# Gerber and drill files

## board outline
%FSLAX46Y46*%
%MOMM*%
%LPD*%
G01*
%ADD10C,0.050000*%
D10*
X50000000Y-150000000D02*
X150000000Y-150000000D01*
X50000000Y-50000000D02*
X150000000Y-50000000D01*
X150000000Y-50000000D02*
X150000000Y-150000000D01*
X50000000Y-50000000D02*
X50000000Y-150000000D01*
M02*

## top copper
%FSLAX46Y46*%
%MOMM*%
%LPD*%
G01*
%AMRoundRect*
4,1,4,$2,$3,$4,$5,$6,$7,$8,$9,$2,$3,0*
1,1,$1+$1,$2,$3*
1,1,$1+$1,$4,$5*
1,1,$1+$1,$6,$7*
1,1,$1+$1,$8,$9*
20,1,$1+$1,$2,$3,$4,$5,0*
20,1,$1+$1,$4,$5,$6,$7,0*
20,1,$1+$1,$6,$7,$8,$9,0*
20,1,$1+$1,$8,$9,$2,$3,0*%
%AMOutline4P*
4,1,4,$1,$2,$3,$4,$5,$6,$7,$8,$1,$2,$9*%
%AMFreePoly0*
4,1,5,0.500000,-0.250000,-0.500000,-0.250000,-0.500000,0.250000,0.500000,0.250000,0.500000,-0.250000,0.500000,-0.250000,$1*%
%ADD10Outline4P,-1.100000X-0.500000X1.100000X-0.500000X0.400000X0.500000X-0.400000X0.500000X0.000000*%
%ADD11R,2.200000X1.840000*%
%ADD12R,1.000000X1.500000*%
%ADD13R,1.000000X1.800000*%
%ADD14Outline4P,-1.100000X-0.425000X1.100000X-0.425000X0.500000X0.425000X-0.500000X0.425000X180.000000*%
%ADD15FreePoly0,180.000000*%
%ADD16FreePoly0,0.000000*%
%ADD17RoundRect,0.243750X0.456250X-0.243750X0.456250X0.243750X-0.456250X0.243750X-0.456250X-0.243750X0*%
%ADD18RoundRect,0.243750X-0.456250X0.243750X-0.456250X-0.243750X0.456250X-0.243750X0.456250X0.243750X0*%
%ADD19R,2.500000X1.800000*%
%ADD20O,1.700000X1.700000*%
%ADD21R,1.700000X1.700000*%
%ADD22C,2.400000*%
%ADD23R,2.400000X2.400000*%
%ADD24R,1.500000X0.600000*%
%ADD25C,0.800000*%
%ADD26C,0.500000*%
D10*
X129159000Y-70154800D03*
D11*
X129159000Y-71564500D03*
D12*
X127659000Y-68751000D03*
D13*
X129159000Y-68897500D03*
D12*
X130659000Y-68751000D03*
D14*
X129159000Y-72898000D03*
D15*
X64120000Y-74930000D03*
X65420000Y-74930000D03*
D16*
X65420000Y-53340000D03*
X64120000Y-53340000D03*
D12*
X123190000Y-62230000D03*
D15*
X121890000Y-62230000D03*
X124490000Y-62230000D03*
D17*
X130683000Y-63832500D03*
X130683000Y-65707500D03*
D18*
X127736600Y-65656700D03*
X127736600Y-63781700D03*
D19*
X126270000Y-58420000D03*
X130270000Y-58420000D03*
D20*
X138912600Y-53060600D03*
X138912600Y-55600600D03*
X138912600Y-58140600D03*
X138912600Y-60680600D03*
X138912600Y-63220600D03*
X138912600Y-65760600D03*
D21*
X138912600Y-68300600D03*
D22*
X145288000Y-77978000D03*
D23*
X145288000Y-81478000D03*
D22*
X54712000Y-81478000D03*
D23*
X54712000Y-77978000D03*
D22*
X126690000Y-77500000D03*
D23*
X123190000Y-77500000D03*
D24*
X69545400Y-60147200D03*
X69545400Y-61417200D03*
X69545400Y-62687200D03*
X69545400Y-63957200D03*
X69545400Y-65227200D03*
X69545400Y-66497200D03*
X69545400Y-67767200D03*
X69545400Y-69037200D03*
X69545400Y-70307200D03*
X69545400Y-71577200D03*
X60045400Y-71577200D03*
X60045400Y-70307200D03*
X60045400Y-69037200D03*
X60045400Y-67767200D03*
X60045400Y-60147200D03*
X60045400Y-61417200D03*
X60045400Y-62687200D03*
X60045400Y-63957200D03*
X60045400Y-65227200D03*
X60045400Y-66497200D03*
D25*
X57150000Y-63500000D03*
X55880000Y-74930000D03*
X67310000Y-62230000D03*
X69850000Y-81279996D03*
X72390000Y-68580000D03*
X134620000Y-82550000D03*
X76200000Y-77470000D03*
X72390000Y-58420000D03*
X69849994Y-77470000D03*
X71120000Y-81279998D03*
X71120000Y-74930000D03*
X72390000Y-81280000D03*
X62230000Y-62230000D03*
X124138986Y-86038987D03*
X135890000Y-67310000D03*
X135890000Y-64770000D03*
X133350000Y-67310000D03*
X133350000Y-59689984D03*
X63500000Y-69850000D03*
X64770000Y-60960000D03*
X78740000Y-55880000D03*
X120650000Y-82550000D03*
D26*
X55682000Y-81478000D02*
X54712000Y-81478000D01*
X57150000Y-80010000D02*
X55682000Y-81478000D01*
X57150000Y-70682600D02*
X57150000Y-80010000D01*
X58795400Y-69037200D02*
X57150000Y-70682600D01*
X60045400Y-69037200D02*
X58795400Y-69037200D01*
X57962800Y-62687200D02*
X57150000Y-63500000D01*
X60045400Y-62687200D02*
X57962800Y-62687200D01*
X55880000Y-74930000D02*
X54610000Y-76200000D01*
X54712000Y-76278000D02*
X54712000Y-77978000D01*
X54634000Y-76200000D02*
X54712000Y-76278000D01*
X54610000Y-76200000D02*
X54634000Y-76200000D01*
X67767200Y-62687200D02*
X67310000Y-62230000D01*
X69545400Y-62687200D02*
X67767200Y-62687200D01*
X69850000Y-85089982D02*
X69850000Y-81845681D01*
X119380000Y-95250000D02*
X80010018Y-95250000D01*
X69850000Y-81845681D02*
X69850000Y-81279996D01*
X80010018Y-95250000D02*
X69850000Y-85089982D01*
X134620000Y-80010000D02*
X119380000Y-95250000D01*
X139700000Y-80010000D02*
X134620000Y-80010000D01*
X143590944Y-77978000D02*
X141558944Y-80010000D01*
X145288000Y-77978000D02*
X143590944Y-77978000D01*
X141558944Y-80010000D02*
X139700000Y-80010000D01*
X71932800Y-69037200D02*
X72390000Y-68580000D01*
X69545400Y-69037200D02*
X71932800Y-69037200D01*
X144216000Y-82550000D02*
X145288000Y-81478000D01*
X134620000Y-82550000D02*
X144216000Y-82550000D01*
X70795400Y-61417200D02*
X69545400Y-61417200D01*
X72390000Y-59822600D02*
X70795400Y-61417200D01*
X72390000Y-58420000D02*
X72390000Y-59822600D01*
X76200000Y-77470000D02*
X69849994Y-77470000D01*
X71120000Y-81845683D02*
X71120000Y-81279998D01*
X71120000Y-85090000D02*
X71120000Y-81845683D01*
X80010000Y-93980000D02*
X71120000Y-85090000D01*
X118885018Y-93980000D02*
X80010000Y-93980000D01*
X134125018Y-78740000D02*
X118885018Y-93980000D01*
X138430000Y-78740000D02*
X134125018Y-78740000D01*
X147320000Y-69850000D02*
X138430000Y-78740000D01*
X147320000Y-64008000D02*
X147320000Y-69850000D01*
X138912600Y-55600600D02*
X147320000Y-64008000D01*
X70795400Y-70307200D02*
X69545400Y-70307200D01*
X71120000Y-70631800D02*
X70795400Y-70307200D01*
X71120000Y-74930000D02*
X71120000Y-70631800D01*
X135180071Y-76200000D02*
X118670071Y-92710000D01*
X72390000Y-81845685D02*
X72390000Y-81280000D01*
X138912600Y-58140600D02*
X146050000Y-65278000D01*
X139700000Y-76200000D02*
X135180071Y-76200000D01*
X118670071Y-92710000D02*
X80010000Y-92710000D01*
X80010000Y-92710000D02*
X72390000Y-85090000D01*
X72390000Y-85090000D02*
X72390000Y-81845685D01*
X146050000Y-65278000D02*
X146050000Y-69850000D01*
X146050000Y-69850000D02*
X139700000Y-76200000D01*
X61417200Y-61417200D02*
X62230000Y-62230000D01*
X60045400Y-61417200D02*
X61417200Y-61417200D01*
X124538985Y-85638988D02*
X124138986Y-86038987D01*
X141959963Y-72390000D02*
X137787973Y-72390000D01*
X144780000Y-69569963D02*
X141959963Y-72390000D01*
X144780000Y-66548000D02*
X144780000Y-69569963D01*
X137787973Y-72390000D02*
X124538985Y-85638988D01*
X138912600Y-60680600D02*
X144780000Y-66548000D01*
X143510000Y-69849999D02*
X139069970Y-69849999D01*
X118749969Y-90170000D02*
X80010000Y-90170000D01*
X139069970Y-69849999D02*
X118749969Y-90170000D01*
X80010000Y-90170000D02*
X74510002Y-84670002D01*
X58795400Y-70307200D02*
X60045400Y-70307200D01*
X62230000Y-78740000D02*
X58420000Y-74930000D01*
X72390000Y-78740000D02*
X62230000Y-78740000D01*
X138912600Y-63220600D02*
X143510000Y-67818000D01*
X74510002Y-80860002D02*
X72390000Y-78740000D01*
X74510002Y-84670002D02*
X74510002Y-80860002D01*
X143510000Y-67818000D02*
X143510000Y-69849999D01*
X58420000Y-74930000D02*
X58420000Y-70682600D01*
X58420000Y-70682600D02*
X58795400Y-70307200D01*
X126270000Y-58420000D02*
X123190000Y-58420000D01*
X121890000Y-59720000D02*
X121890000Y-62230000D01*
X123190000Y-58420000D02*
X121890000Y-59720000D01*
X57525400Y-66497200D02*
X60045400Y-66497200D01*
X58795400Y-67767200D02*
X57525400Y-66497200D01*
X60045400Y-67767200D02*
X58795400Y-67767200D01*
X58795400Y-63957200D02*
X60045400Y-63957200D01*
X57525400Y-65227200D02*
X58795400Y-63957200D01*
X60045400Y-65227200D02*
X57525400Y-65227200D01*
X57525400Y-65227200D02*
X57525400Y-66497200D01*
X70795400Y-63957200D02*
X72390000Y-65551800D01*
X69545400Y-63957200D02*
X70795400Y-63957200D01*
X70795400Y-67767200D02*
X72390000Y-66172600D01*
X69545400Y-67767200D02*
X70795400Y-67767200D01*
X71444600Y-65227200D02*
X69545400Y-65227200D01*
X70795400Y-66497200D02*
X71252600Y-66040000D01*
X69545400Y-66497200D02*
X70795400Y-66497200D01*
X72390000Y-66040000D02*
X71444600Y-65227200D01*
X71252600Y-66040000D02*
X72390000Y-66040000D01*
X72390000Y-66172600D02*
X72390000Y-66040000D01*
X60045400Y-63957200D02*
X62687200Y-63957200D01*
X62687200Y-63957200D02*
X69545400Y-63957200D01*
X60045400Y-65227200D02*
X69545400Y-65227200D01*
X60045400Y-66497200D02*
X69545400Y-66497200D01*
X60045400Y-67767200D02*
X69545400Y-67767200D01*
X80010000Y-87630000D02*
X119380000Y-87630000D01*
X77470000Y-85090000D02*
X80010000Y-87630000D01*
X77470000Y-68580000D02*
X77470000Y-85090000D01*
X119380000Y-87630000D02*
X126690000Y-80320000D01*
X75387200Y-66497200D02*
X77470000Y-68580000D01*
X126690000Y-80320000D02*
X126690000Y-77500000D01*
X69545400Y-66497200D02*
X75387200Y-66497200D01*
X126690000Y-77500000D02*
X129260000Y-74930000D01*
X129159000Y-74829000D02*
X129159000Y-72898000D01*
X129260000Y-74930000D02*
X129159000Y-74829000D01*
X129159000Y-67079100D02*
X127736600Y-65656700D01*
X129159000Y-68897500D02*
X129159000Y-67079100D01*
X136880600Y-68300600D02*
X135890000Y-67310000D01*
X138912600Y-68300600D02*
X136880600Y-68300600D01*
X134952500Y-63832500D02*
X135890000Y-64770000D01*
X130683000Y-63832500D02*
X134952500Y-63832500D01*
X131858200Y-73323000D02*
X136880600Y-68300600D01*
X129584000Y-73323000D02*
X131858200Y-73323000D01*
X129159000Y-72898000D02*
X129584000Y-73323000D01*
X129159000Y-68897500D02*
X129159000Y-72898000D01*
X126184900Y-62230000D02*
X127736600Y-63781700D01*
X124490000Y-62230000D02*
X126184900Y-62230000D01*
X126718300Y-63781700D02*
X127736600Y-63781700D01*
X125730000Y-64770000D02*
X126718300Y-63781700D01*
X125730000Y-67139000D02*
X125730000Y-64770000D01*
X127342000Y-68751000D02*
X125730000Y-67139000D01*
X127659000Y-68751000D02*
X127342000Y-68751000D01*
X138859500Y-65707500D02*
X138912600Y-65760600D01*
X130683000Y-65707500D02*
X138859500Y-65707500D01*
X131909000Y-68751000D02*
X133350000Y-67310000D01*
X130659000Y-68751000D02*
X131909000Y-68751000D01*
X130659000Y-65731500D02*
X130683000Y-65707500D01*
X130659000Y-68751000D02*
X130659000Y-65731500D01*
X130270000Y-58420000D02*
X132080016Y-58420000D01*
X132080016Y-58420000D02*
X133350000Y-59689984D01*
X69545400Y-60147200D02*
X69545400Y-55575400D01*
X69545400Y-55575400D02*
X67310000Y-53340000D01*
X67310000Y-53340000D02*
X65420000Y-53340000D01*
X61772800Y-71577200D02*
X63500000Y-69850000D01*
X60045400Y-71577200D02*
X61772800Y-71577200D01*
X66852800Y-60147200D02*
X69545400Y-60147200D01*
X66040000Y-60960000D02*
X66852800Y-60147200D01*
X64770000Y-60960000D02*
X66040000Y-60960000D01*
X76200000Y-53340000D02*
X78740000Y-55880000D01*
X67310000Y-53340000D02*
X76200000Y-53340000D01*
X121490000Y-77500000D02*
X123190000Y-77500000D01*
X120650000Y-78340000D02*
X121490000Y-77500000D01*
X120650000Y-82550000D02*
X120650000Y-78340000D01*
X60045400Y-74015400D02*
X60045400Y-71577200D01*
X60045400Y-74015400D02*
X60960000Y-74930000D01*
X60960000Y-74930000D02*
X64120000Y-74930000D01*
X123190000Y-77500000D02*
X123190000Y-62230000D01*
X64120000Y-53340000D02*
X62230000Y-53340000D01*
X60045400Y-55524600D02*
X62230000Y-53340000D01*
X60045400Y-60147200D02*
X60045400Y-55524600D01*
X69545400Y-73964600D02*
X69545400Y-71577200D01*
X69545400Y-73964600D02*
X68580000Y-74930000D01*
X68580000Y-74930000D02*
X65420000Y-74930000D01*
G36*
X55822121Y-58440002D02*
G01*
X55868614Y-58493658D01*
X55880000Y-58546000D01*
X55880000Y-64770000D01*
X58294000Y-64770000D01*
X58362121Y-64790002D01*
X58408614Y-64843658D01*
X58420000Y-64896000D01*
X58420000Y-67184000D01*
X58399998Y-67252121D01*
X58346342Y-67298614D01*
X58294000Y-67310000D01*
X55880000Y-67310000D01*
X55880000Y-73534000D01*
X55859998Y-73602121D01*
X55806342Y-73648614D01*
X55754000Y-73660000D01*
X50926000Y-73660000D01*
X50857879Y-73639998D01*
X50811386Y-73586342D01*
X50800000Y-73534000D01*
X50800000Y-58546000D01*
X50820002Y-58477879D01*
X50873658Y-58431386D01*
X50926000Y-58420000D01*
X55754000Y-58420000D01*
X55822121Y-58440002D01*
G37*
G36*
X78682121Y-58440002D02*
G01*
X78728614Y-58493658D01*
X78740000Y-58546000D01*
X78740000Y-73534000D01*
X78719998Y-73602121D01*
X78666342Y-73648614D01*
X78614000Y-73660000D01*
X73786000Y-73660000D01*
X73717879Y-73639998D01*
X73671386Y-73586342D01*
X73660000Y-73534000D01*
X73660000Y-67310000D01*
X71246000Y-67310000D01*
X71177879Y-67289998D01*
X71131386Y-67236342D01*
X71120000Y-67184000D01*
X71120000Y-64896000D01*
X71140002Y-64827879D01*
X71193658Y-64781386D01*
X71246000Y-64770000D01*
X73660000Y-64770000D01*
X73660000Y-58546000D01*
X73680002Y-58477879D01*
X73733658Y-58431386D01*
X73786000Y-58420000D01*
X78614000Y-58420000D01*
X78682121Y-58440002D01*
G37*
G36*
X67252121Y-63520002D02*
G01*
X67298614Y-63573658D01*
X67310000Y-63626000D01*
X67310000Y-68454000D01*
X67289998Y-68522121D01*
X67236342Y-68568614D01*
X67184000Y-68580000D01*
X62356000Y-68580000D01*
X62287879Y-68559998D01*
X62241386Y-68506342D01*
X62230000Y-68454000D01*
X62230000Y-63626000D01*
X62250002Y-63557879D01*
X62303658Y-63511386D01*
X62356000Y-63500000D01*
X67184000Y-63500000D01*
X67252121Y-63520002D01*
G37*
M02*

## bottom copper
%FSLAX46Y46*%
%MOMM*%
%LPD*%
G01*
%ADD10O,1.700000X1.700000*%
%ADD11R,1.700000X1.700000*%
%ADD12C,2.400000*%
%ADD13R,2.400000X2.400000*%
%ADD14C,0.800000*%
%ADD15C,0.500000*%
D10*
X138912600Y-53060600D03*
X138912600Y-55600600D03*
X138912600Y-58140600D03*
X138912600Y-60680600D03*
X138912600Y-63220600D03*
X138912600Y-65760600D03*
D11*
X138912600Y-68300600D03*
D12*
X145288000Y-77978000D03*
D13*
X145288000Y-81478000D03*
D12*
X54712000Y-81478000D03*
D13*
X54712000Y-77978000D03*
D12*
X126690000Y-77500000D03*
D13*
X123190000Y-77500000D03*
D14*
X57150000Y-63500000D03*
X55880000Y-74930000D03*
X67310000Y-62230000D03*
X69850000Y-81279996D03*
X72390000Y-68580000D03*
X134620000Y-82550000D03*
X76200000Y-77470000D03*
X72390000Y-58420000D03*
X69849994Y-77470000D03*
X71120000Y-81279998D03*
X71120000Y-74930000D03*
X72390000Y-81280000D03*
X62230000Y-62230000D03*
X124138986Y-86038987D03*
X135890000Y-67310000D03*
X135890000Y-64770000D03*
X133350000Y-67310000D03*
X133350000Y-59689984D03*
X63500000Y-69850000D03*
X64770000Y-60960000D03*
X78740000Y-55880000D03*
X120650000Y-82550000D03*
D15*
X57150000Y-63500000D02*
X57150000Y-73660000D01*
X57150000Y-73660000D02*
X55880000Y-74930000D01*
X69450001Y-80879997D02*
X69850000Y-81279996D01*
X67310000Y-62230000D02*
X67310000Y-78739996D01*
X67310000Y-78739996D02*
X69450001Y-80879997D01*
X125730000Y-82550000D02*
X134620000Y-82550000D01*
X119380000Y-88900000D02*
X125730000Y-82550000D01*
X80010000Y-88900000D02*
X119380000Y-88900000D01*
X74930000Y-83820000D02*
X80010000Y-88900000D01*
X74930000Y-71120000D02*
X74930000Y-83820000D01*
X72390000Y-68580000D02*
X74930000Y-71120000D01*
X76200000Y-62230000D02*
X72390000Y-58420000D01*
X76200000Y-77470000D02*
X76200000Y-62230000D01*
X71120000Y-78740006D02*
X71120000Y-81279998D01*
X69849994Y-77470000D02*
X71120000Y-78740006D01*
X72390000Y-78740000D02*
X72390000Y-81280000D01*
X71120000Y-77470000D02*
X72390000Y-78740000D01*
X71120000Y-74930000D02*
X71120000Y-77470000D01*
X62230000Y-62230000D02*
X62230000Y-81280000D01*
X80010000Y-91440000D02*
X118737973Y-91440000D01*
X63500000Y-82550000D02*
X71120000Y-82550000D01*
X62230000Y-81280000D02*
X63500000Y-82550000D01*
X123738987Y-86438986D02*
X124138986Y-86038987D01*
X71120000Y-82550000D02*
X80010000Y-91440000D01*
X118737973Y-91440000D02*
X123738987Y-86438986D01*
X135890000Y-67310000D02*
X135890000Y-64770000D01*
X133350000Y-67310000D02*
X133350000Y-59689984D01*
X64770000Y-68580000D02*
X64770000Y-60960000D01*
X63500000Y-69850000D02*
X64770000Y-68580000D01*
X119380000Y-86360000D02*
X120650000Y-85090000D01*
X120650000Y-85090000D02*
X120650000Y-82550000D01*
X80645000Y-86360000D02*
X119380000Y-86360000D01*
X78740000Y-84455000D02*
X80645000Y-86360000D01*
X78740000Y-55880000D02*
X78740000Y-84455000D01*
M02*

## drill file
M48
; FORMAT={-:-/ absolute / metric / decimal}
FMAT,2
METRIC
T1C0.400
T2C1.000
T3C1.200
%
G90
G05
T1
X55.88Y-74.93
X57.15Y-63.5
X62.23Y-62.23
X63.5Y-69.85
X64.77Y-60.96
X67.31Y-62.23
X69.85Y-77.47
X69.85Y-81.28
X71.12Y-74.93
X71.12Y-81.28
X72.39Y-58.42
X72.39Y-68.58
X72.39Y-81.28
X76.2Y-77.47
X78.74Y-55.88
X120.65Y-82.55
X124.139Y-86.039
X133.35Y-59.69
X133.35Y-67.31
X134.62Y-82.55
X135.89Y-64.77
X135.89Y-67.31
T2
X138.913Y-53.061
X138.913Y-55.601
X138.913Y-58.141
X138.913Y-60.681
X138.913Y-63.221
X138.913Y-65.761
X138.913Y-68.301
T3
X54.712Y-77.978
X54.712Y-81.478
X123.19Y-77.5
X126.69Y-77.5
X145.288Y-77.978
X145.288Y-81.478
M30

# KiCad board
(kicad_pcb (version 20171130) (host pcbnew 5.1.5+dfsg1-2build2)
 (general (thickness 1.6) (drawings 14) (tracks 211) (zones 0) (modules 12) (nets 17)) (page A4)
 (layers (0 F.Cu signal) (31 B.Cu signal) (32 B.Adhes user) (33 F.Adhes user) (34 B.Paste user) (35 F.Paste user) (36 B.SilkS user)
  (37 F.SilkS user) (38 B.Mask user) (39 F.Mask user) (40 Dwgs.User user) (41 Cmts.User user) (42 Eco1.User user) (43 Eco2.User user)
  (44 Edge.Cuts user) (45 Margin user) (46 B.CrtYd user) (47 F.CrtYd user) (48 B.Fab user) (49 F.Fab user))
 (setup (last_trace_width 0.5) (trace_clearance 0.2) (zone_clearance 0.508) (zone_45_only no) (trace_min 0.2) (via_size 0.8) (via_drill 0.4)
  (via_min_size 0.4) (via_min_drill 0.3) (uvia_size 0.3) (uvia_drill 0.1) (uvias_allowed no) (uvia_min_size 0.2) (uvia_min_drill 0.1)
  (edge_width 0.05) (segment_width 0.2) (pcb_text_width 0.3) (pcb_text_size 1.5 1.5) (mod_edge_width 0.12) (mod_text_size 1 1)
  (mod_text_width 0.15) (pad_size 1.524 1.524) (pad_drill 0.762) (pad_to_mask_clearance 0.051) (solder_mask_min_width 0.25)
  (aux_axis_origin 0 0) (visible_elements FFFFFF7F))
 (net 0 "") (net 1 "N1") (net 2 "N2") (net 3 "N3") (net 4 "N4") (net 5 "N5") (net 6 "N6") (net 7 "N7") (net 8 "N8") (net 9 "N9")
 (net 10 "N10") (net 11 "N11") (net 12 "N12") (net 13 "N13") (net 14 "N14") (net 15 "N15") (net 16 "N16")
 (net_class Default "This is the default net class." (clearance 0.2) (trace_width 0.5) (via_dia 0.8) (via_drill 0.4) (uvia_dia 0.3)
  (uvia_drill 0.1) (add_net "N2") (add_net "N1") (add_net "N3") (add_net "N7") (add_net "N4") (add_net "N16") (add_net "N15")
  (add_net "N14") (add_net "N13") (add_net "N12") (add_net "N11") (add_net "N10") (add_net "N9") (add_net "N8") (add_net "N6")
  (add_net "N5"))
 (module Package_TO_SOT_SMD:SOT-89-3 (layer F.Cu) (at 129.159 70.231 270)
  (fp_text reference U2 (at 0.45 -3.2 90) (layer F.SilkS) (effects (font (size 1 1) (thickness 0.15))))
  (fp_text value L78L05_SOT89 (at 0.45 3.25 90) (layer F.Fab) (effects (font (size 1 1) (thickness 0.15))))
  (pad 2 smd trapezoid (at -0.0762 0) (size 1.5 1) (rect_delta 0 0.7) (layers F.Cu F.Paste F.Mask) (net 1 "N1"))
  (pad 2 smd rect (at 1.3335 0 180) (size 2.2 1.84) (layers F.Cu F.Paste F.Mask) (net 1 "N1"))
  (pad 3 smd rect (at -1.48 1.5 180) (size 1 1.5) (layers F.Cu F.Paste F.Mask) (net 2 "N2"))
  (pad 2 smd rect (at -1.3335 0 180) (size 1 1.8) (layers F.Cu F.Paste F.Mask) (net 1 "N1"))
  (pad 1 smd rect (at -1.48 -1.5 180) (size 1 1.5) (layers F.Cu F.Paste F.Mask) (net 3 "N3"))
  (pad 2 smd trapezoid (at 2.667 0 180) (size 1.6 0.85) (rect_delta 0 0.6) (layers F.Cu F.Paste F.Mask) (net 1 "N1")))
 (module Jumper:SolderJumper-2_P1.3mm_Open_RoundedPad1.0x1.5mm (layer F.Cu) (at 64.77 74.93 180)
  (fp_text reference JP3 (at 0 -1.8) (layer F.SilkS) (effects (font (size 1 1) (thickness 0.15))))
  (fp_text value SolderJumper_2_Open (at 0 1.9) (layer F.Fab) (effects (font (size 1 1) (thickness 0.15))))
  (pad 2 smd custom (at 0.65 0 180) (size 1 0.5) (layers F.Cu F.Mask) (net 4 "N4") (zone_connect 2)
   (options (clearance outline) (anchor rect)) (primitives))
  (pad 1 smd custom (at -0.65 0 180) (size 1 0.5) (layers F.Cu F.Mask) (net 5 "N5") (zone_connect 2)
   (options (clearance outline) (anchor rect)) (primitives)))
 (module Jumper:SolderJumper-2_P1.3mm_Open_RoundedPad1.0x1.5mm (layer F.Cu) (at 64.77 53.34)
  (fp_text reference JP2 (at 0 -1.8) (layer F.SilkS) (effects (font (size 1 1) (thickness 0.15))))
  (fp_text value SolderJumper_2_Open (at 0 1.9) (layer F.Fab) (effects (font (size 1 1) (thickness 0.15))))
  (pad 2 smd custom (at 0.65 0) (size 1 0.5) (layers F.Cu F.Mask) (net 4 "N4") (zone_connect 2) (options (clearance outline) (anchor rect))
   (primitives))
  (pad 1 smd custom (at -0.65 0) (size 1 0.5) (layers F.Cu F.Mask) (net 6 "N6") (zone_connect 2) (options (clearance outline) (anchor rect))
   (primitives)))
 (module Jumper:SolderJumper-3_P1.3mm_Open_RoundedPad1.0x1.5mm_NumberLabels (layer F.Cu) (at 123.19 62.23 180)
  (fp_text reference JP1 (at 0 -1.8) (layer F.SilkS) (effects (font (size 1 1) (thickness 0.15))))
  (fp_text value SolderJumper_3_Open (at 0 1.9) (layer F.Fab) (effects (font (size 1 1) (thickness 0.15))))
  (pad 2 smd rect (at 0 0 180) (size 1 1.5) (layers F.Cu F.Mask) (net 4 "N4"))
  (pad 3 smd custom (at 1.3 0 180) (size 1 0.5) (layers F.Cu F.Mask) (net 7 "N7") (zone_connect 2)
   (options (clearance outline) (anchor rect)) (primitives))
  (pad 1 smd custom (at -1.3 0 180) (size 1 0.5) (layers F.Cu F.Mask) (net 2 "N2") (zone_connect 2)
   (options (clearance outline) (anchor rect)) (primitives)))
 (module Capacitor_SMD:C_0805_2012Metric (layer F.Cu) (at 130.683 64.77 90)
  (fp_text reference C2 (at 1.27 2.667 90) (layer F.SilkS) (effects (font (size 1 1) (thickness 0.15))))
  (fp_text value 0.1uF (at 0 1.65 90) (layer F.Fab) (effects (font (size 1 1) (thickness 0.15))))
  (pad 2 smd roundrect (at 0.9375 0 90) (size 0.975 1.4) (layers F.Cu F.Paste F.Mask) (roundrect_rratio 0.25) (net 1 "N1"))
  (pad 1 smd roundrect (at -0.9375 0 90) (size 0.975 1.4) (layers F.Cu F.Paste F.Mask) (roundrect_rratio 0.25) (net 3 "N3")))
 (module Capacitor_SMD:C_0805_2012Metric (layer F.Cu) (at 127.7366 64.7192 270)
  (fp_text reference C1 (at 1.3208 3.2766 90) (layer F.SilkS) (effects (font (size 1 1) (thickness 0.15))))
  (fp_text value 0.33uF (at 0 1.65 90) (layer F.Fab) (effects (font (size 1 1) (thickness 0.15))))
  (pad 2 smd roundrect (at 0.9375 0 270) (size 0.975 1.4) (layers F.Cu F.Paste F.Mask) (roundrect_rratio 0.25) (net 1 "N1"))
  (pad 1 smd roundrect (at -0.9375 0 270) (size 0.975 1.4) (layers F.Cu F.Paste F.Mask) (roundrect_rratio 0.25) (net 2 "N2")))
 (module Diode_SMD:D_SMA (layer F.Cu) (at 128.27 58.42 180)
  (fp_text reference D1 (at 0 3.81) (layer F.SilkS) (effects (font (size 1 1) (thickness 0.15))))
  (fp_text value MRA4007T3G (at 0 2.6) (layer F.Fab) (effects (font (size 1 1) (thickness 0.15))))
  (pad 2 smd rect (at 2 0 180) (size 2.5 1.8) (layers F.Cu F.Paste F.Mask) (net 7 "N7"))
  (pad 1 smd rect (at -2 0 180) (size 2.5 1.8) (layers F.Cu F.Paste F.Mask) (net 3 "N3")))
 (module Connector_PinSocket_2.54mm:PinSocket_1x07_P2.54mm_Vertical (layer F.Cu) (at 138.9126 68.3006 180)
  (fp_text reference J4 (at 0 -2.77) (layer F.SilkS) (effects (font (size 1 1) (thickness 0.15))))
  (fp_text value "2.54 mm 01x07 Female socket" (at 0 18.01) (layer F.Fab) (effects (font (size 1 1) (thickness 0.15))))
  (pad 7 thru_hole oval (at 0 15.24 180) (size 1.7 1.7) (drill 1) (layers *.Cu *.Mask) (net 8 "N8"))
  (pad 6 thru_hole oval (at 0 12.7 180) (size 1.7 1.7) (drill 1) (layers *.Cu *.Mask) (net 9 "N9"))
  (pad 5 thru_hole oval (at 0 10.16 180) (size 1.7 1.7) (drill 1) (layers *.Cu *.Mask) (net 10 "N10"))
  (pad 4 thru_hole oval (at 0 7.62 180) (size 1.7 1.7) (drill 1) (layers *.Cu *.Mask) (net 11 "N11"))
  (pad 3 thru_hole oval (at 0 5.08 180) (size 1.7 1.7) (drill 1) (layers *.Cu *.Mask) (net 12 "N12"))
  (pad 2 thru_hole oval (at 0 2.54 180) (size 1.7 1.7) (drill 1) (layers *.Cu *.Mask) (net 3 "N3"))
  (pad 1 thru_hole rect (at 0 0 180) (size 1.7 1.7) (drill 1) (layers *.Cu *.Mask) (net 1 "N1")))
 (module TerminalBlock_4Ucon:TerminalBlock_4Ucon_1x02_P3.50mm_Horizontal (layer F.Cu) (at 145.288 81.478 90)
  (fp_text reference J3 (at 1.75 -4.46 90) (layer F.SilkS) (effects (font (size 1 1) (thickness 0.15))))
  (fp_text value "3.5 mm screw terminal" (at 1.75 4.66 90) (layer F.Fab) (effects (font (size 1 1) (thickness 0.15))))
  (pad 2 thru_hole circle (at 3.5 0 90) (size 2.4 2.4) (drill 1.2) (layers *.Cu *.Mask) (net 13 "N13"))
  (pad 1 thru_hole rect (at 0 0 90) (size 2.4 2.4) (drill 1.2) (layers *.Cu *.Mask) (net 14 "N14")))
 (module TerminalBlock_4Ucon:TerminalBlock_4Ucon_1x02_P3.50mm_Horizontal (layer F.Cu) (at 54.712 77.978 270)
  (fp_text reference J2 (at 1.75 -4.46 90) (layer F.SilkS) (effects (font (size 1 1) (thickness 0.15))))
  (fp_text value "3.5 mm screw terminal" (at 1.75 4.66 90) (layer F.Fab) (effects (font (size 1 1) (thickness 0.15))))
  (pad 2 thru_hole circle (at 3.5 0 270) (size 2.4 2.4) (drill 1.2) (layers *.Cu *.Mask) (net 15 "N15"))
  (pad 1 thru_hole rect (at 0 0 270) (size 2.4 2.4) (drill 1.2) (layers *.Cu *.Mask) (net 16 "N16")))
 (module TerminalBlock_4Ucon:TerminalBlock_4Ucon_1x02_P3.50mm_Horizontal (layer F.Cu) (at 123.19 77.5)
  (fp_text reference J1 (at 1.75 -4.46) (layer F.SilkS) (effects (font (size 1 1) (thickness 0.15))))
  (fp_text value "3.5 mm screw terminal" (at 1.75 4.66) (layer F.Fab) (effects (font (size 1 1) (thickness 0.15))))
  (pad 2 thru_hole circle (at 3.5 0) (size 2.4 2.4) (drill 1.2) (layers *.Cu *.Mask) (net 1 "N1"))
  (pad 1 thru_hole rect (at 0 0) (size 2.4 2.4) (drill 1.2) (layers *.Cu *.Mask) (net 4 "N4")))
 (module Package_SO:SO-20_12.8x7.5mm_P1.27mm (layer F.Cu) (at 64.7954 65.8622)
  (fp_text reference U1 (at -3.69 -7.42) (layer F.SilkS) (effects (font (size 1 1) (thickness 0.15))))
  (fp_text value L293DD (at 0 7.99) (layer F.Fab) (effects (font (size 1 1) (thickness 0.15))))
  (pad 20 smd rect (at 4.75 -5.715) (size 1.5 0.6) (layers F.Cu F.Paste F.Mask) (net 4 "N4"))
  (pad 19 smd rect (at 4.75 -4.445) (size 1.5 0.6) (layers F.Cu F.Paste F.Mask) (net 9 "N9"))
  (pad 18 smd rect (at 4.75 -3.175) (size 1.5 0.6) (layers F.Cu F.Paste F.Mask) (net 13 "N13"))
  (pad 17 smd rect (at 4.75 -1.905) (size 1.5 0.6) (layers F.Cu F.Paste F.Mask) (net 1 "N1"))
  (pad 16 smd rect (at 4.75 -0.635) (size 1.5 0.6) (layers F.Cu F.Paste F.Mask) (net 1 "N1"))
  (pad 15 smd rect (at 4.75 0.635) (size 1.5 0.6) (layers F.Cu F.Paste F.Mask) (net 1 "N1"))
  (pad 14 smd rect (at 4.75 1.905) (size 1.5 0.6) (layers F.Cu F.Paste F.Mask) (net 1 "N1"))
  (pad 13 smd rect (at 4.75 3.175) (size 1.5 0.6) (layers F.Cu F.Paste F.Mask) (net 14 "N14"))
  (pad 12 smd rect (at 4.75 4.445) (size 1.5 0.6) (layers F.Cu F.Paste F.Mask) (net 10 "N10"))
  (pad 11 smd rect (at 4.75 5.715) (size 1.5 0.6) (layers F.Cu F.Paste F.Mask) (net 5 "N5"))
  (pad 10 smd rect (at -4.75 5.715) (size 1.5 0.6) (layers F.Cu F.Paste F.Mask) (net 4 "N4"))
  (pad 9 smd rect (at -4.75 4.445) (size 1.5 0.6) (layers F.Cu F.Paste F.Mask) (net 12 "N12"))
  (pad 8 smd rect (at -4.75 3.175) (size 1.5 0.6) (layers F.Cu F.Paste F.Mask) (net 15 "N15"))
  (pad 7 smd rect (at -4.75 1.905) (size 1.5 0.6) (layers F.Cu F.Paste F.Mask) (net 1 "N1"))
  (pad 1 smd rect (at -4.75 -5.715) (size 1.5 0.6) (layers F.Cu F.Paste F.Mask) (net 6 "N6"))
  (pad 2 smd rect (at -4.75 -4.445) (size 1.5 0.6) (layers F.Cu F.Paste F.Mask) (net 11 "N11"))
  (pad 3 smd rect (at -4.75 -3.175) (size 1.5 0.6) (layers F.Cu F.Paste F.Mask) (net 16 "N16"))
  (pad 4 smd rect (at -4.75 -1.905) (size 1.5 0.6) (layers F.Cu F.Paste F.Mask) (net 1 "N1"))
  (pad 5 smd rect (at -4.75 -0.635) (size 1.5 0.6) (layers F.Cu F.Paste F.Mask) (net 1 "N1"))
  (pad 6 smd rect (at -4.75 0.635) (size 1.5 0.6) (layers F.Cu F.Paste F.Mask) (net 1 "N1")))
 (gr_line (start 50 150) (end 150 150) (layer Edge.Cuts) (width 0.05))
 (gr_line (start 50 50) (end 150 50) (layer Edge.Cuts) (width 0.05))
 (gr_line (start 150 50) (end 150 150) (layer Edge.Cuts) (width 0.05))
 (gr_line (start 50 50) (end 50 150) (layer Edge.Cuts) (width 0.05))
 (segment (start 55.682 81.478) (end 54.712 81.478) (width 0.5) (layer F.Cu) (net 15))
 (segment (start 57.15 80.01) (end 55.682 81.478) (width 0.5) (layer F.Cu) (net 15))
 (segment (start 57.15 70.6826) (end 57.15 80.01) (width 0.5) (layer F.Cu) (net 15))
 (segment (start 58.7954 69.0372) (end 57.15 70.6826) (width 0.5) (layer F.Cu) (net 15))
 (segment (start 60.0454 69.0372) (end 58.7954 69.0372) (width 0.5) (layer F.Cu) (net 15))
 (via (at 57.15 63.5) (size 0.8) (drill 0.4) (layers F.Cu B.Cu) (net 16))
 (segment (start 57.9628 62.6872) (end 57.15 63.5) (width 0.5) (layer F.Cu) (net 16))
 (segment (start 60.0454 62.6872) (end 57.9628 62.6872) (width 0.5) (layer F.Cu) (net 16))
 (segment (start 57.15 63.5) (end 57.15 73.66) (width 0.5) (layer B.Cu) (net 16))
 (via (at 55.88 74.93) (size 0.8) (drill 0.4) (layers F.Cu B.Cu) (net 16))
 (segment (start 57.15 73.66) (end 55.88 74.93) (width 0.5) (layer B.Cu) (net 16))
 (segment (start 55.88 74.93) (end 54.61 76.2) (width 0.5) (layer F.Cu) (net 16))
 (segment (start 54.712 76.278) (end 54.712 77.978) (width 0.5) (layer F.Cu) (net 16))
 (segment (start 54.634 76.2) (end 54.712 76.278) (width 0.5) (layer F.Cu) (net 16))
 (segment (start 54.61 76.2) (end 54.634 76.2) (width 0.5) (layer F.Cu) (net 16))
 (via (at 67.31 62.23) (size 0.8) (drill 0.4) (layers F.Cu B.Cu) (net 13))
 (segment (start 67.7672 62.6872) (end 67.31 62.23) (width 0.5) (layer F.Cu) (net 13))
 (segment (start 69.5454 62.6872) (end 67.7672 62.6872) (width 0.5) (layer F.Cu) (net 13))
 (via (at 69.85 81.279996) (size 0.8) (drill 0.4) (layers F.Cu B.Cu) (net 13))
 (segment (start 69.450001 80.879997) (end 69.85 81.279996) (width 0.5) (layer B.Cu) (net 13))
 (segment (start 67.31 62.23) (end 67.31 78.739996) (width 0.5) (layer B.Cu) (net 13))
 (segment (start 67.31 78.739996) (end 69.450001 80.879997) (width 0.5) (layer B.Cu) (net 13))
 (segment (start 69.85 85.089982) (end 69.85 81.845681) (width 0.5) (layer F.Cu) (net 13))
 (segment (start 119.38 95.25) (end 80.010018 95.25) (width 0.5) (layer F.Cu) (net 13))
 (segment (start 69.85 81.845681) (end 69.85 81.279996) (width 0.5) (layer F.Cu) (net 13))
 (segment (start 80.010018 95.25) (end 69.85 85.089982) (width 0.5) (layer F.Cu) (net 13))
 (segment (start 134.62 80.01) (end 119.38 95.25) (width 0.5) (layer F.Cu) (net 13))
 (segment (start 139.7 80.01) (end 134.62 80.01) (width 0.5) (layer F.Cu) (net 13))
 (segment (start 143.590944 77.978) (end 141.558944 80.01) (width 0.5) (layer F.Cu) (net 13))
 (segment (start 145.288 77.978) (end 143.590944 77.978) (width 0.5) (layer F.Cu) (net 13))
 (segment (start 141.558944 80.01) (end 139.7 80.01) (width 0.5) (layer F.Cu) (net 13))
 (via (at 72.39 68.58) (size 0.8) (drill 0.4) (layers F.Cu B.Cu) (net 14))
 (segment (start 71.9328 69.0372) (end 72.39 68.58) (width 0.5) (layer F.Cu) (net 14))
 (segment (start 69.5454 69.0372) (end 71.9328 69.0372) (width 0.5) (layer F.Cu) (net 14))
 (via (at 134.62 82.55) (size 0.8) (drill 0.4) (layers F.Cu B.Cu) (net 14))
 (segment (start 144.216 82.55) (end 145.288 81.478) (width 0.5) (layer F.Cu) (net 14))
 (segment (start 134.62 82.55) (end 144.216 82.55) (width 0.5) (layer F.Cu) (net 14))
 (segment (start 125.73 82.55) (end 134.62 82.55) (width 0.5) (layer B.Cu) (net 14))
 (segment (start 119.38 88.9) (end 125.73 82.55) (width 0.5) (layer B.Cu) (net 14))
 (segment (start 80.01 88.9) (end 119.38 88.9) (width 0.5) (layer B.Cu) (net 14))
 (segment (start 74.93 83.82) (end 80.01 88.9) (width 0.5) (layer B.Cu) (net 14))
 (segment (start 74.93 71.12) (end 74.93 83.82) (width 0.5) (layer B.Cu) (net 14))
 (segment (start 72.39 68.58) (end 74.93 71.12) (width 0.5) (layer B.Cu) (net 14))
 (via (at 76.2 77.47) (size 0.8) (drill 0.4) (layers F.Cu B.Cu) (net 9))
 (via (at 72.39 58.42) (size 0.8) (drill 0.4) (layers F.Cu B.Cu) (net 9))
 (segment (start 76.2 62.23) (end 72.39 58.42) (width 0.5) (layer B.Cu) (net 9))
 (segment (start 76.2 77.47) (end 76.2 62.23) (width 0.5) (layer B.Cu) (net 9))
 (segment (start 70.7954 61.4172) (end 69.5454 61.4172) (width 0.5) (layer F.Cu) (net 9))
 (segment (start 72.39 59.8226) (end 70.7954 61.4172) (width 0.5) (layer F.Cu) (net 9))
 (segment (start 72.39 58.42) (end 72.39 59.8226) (width 0.5) (layer F.Cu) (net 9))
 (via (at 69.849994 77.47) (size 0.8) (drill 0.4) (layers F.Cu B.Cu) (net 9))
 (segment (start 76.2 77.47) (end 69.849994 77.47) (width 0.5) (layer F.Cu) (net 9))
 (segment (start 71.12 78.740006) (end 71.12 81.279998) (width 0.5) (layer B.Cu) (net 9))
 (segment (start 69.849994 77.47) (end 71.12 78.740006) (width 0.5) (layer B.Cu) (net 9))
 (via (at 71.12 81.279998) (size 0.8) (drill 0.4) (layers F.Cu B.Cu) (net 9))
 (segment (start 71.12 81.845683) (end 71.12 81.279998) (width 0.5) (layer F.Cu) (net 9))
 (segment (start 71.12 85.09) (end 71.12 81.845683) (width 0.5) (layer F.Cu) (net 9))
 (segment (start 80.01 93.98) (end 71.12 85.09) (width 0.5) (layer F.Cu) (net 9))
 (segment (start 118.885018 93.98) (end 80.01 93.98) (width 0.5) (layer F.Cu) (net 9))
 (segment (start 134.125018 78.74) (end 118.885018 93.98) (width 0.5) (layer F.Cu) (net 9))
 (segment (start 138.43 78.74) (end 134.125018 78.74) (width 0.5) (layer F.Cu) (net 9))
 (segment (start 147.32 69.85) (end 138.43 78.74) (width 0.5) (layer F.Cu) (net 9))
 (segment (start 147.32 64.008) (end 147.32 69.85) (width 0.5) (layer F.Cu) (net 9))
 (segment (start 138.9126 55.6006) (end 147.32 64.008) (width 0.5) (layer F.Cu) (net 9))
 (via (at 71.12 74.93) (size 0.8) (drill 0.4) (layers F.Cu B.Cu) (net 10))
 (segment (start 70.7954 70.3072) (end 69.5454 70.3072) (width 0.5) (layer F.Cu) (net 10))
 (segment (start 71.12 70.6318) (end 70.7954 70.3072) (width 0.5) (layer F.Cu) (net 10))
 (segment (start 71.12 74.93) (end 71.12 70.6318) (width 0.5) (layer F.Cu) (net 10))
 (via (at 72.39 81.28) (size 0.8) (drill 0.4) (layers F.Cu B.Cu) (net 10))
 (segment (start 72.39 78.74) (end 72.39 81.28) (width 0.5) (layer B.Cu) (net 10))
 (segment (start 71.12 77.47) (end 72.39 78.74) (width 0.5) (layer B.Cu) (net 10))
 (segment (start 71.12 74.93) (end 71.12 77.47) (width 0.5) (layer B.Cu) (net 10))
 (segment (start 135.180071 76.2) (end 118.670071 92.71) (width 0.5) (layer F.Cu) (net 10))
 (segment (start 72.39 81.845685) (end 72.39 81.28) (width 0.5) (layer F.Cu) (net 10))
 (segment (start 138.9126 58.1406) (end 146.05 65.278) (width 0.5) (layer F.Cu) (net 10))
 (segment (start 139.7 76.2) (end 135.180071 76.2) (width 0.5) (layer F.Cu) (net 10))
 (segment (start 118.670071 92.71) (end 80.01 92.71) (width 0.5) (layer F.Cu) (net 10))
 (segment (start 80.01 92.71) (end 72.39 85.09) (width 0.5) (layer F.Cu) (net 10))
 (segment (start 72.39 85.09) (end 72.39 81.845685) (width 0.5) (layer F.Cu) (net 10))
 (segment (start 146.05 65.278) (end 146.05 69.85) (width 0.5) (layer F.Cu) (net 10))
 (segment (start 146.05 69.85) (end 139.7 76.2) (width 0.5) (layer F.Cu) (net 10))
 (via (at 62.23 62.23) (size 0.8) (drill 0.4) (layers F.Cu B.Cu) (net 11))
 (segment (start 61.4172 61.4172) (end 62.23 62.23) (width 0.5) (layer F.Cu) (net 11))
 (segment (start 60.0454 61.4172) (end 61.4172 61.4172) (width 0.5) (layer F.Cu) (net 11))
 (via (at 124.138986 86.038987) (size 0.8) (drill 0.4) (layers F.Cu B.Cu) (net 11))
 (segment (start 62.23 62.23) (end 62.23 81.28) (width 0.5) (layer B.Cu) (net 11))
 (segment (start 80.01 91.44) (end 118.737973 91.44) (width 0.5) (layer B.Cu) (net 11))
 (segment (start 63.5 82.55) (end 71.12 82.55) (width 0.5) (layer B.Cu) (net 11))
 (segment (start 62.23 81.28) (end 63.5 82.55) (width 0.5) (layer B.Cu) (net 11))
 (segment (start 123.738987 86.438986) (end 124.138986 86.038987) (width 0.5) (layer B.Cu) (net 11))
 (segment (start 71.12 82.55) (end 80.01 91.44) (width 0.5) (layer B.Cu) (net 11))
 (segment (start 118.737973 91.44) (end 123.738987 86.438986) (width 0.5) (layer B.Cu) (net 11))
 (segment (start 124.538985 85.638988) (end 124.138986 86.038987) (width 0.5) (layer F.Cu) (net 11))
 (segment (start 141.959963 72.39) (end 137.787973 72.39) (width 0.5) (layer F.Cu) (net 11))
 (segment (start 144.78 69.569963) (end 141.959963 72.39) (width 0.5) (layer F.Cu) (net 11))
 (segment (start 144.78 66.548) (end 144.78 69.569963) (width 0.5) (layer F.Cu) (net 11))
 (segment (start 137.787973 72.39) (end 124.538985 85.638988) (width 0.5) (layer F.Cu) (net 11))
 (segment (start 138.9126 60.6806) (end 144.78 66.548) (width 0.5) (layer F.Cu) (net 11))
 (segment (start 143.51 69.849999) (end 139.06997 69.849999) (width 0.5) (layer F.Cu) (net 12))
 (segment (start 118.749969 90.17) (end 80.01 90.17) (width 0.5) (layer F.Cu) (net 12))
 (segment (start 139.06997 69.849999) (end 118.749969 90.17) (width 0.5) (layer F.Cu) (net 12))
 (segment (start 80.01 90.17) (end 74.510002 84.670002) (width 0.5) (layer F.Cu) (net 12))
 (segment (start 58.7954 70.3072) (end 60.0454 70.3072) (width 0.5) (layer F.Cu) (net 12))
 (segment (start 62.23 78.74) (end 58.42 74.93) (width 0.5) (layer F.Cu) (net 12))
 (segment (start 72.39 78.74) (end 62.23 78.74) (width 0.5) (layer F.Cu) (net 12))
 (segment (start 138.9126 63.2206) (end 143.51 67.818) (width 0.5) (layer F.Cu) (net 12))
 (segment (start 74.510002 80.860002) (end 72.39 78.74) (width 0.5) (layer F.Cu) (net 12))
 (segment (start 74.510002 84.670002) (end 74.510002 80.860002) (width 0.5) (layer F.Cu) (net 12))
 (segment (start 143.51 67.818) (end 143.51 69.849999) (width 0.5) (layer F.Cu) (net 12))
 (segment (start 58.42 74.93) (end 58.42 70.6826) (width 0.5) (layer F.Cu) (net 12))
 (segment (start 58.42 70.6826) (end 58.7954 70.3072) (width 0.5) (layer F.Cu) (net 12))
 (segment (start 126.27 58.42) (end 123.19 58.42) (width 0.5) (layer F.Cu) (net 7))
 (segment (start 121.89 59.72) (end 121.89 62.23) (width 0.5) (layer F.Cu) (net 7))
 (segment (start 123.19 58.42) (end 121.89 59.72) (width 0.5) (layer F.Cu) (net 7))
 (segment (start 57.5254 66.4972) (end 60.0454 66.4972) (width 0.5) (layer F.Cu) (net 1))
 (segment (start 58.7954 67.7672) (end 57.5254 66.4972) (width 0.5) (layer F.Cu) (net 1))
 (segment (start 60.0454 67.7672) (end 58.7954 67.7672) (width 0.5) (layer F.Cu) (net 1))
 (segment (start 58.7954 63.9572) (end 60.0454 63.9572) (width 0.5) (layer F.Cu) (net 1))
 (segment (start 57.5254 65.2272) (end 58.7954 63.9572) (width 0.5) (layer F.Cu) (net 1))
 (segment (start 60.0454 65.2272) (end 57.5254 65.2272) (width 0.5) (layer F.Cu) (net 1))
 (segment (start 57.5254 65.2272) (end 57.5254 66.4972) (width 0.5) (layer F.Cu) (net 1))
 (segment (start 70.7954 63.9572) (end 72.39 65.5518) (width 0.5) (layer F.Cu) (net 1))
 (segment (start 69.5454 63.9572) (end 70.7954 63.9572) (width 0.5) (layer F.Cu) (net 1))
 (segment (start 70.7954 67.7672) (end 72.39 66.1726) (width 0.5) (layer F.Cu) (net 1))
 (segment (start 69.5454 67.7672) (end 70.7954 67.7672) (width 0.5) (layer F.Cu) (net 1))
 (segment (start 71.4446 65.2272) (end 69.5454 65.2272) (width 0.5) (layer F.Cu) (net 1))
 (segment (start 70.7954 66.4972) (end 71.2526 66.04) (width 0.5) (layer F.Cu) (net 1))
 (segment (start 69.5454 66.4972) (end 70.7954 66.4972) (width 0.5) (layer F.Cu) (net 1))
 (segment (start 72.39 66.04) (end 71.4446 65.2272) (width 0.5) (layer F.Cu) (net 1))
 (segment (start 71.2526 66.04) (end 72.39 66.04) (width 0.5) (layer F.Cu) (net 1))
 (segment (start 72.39 66.1726) (end 72.39 66.04) (width 0.5) (layer F.Cu) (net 1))
 (segment (start 60.0454 63.9572) (end 62.6872 63.9572) (width 0.5) (layer F.Cu) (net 1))
 (segment (start 62.6872 63.9572) (end 69.5454 63.9572) (width 0.5) (layer F.Cu) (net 1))
 (segment (start 60.0454 65.2272) (end 69.5454 65.2272) (width 0.5) (layer F.Cu) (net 1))
 (segment (start 60.0454 66.4972) (end 69.5454 66.4972) (width 0.5) (layer F.Cu) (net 1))
 (segment (start 60.0454 67.7672) (end 69.5454 67.7672) (width 0.5) (layer F.Cu) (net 1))
 (segment (start 80.01 87.63) (end 119.38 87.63) (width 0.5) (layer F.Cu) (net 1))
 (segment (start 77.47 85.09) (end 80.01 87.63) (width 0.5) (layer F.Cu) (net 1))
 (segment (start 77.47 68.58) (end 77.47 85.09) (width 0.5) (layer F.Cu) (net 1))
 (segment (start 119.38 87.63) (end 126.69 80.32) (width 0.5) (layer F.Cu) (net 1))
 (segment (start 75.3872 66.4972) (end 77.47 68.58) (width 0.5) (layer F.Cu) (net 1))
 (segment (start 126.69 80.32) (end 126.69 77.5) (width 0.5) (layer F.Cu) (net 1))
 (segment (start 69.5454 66.4972) (end 75.3872 66.4972) (width 0.5) (layer F.Cu) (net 1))
 (segment (start 126.69 77.5) (end 129.26 74.93) (width 0.5) (layer F.Cu) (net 1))
 (segment (start 129.159 74.829) (end 129.159 72.898) (width 0.5) (layer F.Cu) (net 1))
 (segment (start 129.26 74.93) (end 129.159 74.829) (width 0.5) (layer F.Cu) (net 1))
 (segment (start 129.159 67.0791) (end 127.7366 65.6567) (width 0.5) (layer F.Cu) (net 1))
 (segment (start 129.159 68.8975) (end 129.159 67.0791) (width 0.5) (layer F.Cu) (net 1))
 (via (at 135.89 67.31) (size 0.8) (drill 0.4) (layers F.Cu B.Cu) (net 1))
 (segment (start 136.8806 68.3006) (end 135.89 67.31) (width 0.5) (layer F.Cu) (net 1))
 (segment (start 138.9126 68.3006) (end 136.8806 68.3006) (width 0.5) (layer F.Cu) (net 1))
 (via (at 135.89 64.77) (size 0.8) (drill 0.4) (layers F.Cu B.Cu) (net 1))
 (segment (start 135.89 67.31) (end 135.89 64.77) (width 0.5) (layer B.Cu) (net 1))
 (segment (start 134.9525 63.8325) (end 135.89 64.77) (width 0.5) (layer F.Cu) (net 1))
 (segment (start 130.683 63.8325) (end 134.9525 63.8325) (width 0.5) (layer F.Cu) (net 1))
 (segment (start 131.8582 73.323) (end 136.8806 68.3006) (width 0.5) (layer F.Cu) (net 1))
 (segment (start 129.584 73.323) (end 131.8582 73.323) (width 0.5) (layer F.Cu) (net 1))
 (segment (start 129.159 72.898) (end 129.584 73.323) (width 0.5) (layer F.Cu) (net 1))
 (segment (start 129.159 68.8975) (end 129.159 72.898) (width 0.5) (layer F.Cu) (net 1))
 (segment (start 126.1849 62.23) (end 127.7366 63.7817) (width 0.5) (layer F.Cu) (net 2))
 (segment (start 124.49 62.23) (end 126.1849 62.23) (width 0.5) (layer F.Cu) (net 2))
 (segment (start 126.7183 63.7817) (end 127.7366 63.7817) (width 0.5) (layer F.Cu) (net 2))
 (segment (start 125.73 64.77) (end 126.7183 63.7817) (width 0.5) (layer F.Cu) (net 2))
 (segment (start 125.73 67.139) (end 125.73 64.77) (width 0.5) (layer F.Cu) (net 2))
 (segment (start 127.342 68.751) (end 125.73 67.139) (width 0.5) (layer F.Cu) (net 2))
 (segment (start 127.659 68.751) (end 127.342 68.751) (width 0.5) (layer F.Cu) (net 2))
 (segment (start 138.8595 65.7075) (end 138.9126 65.7606) (width 0.5) (layer F.Cu) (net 3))
 (segment (start 130.683 65.7075) (end 138.8595 65.7075) (width 0.5) (layer F.Cu) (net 3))
 (via (at 133.35 67.31) (size 0.8) (drill 0.4) (layers F.Cu B.Cu) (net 3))
 (segment (start 131.909 68.751) (end 133.35 67.31) (width 0.5) (layer F.Cu) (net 3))
 (segment (start 130.659 68.751) (end 131.909 68.751) (width 0.5) (layer F.Cu) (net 3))
 (segment (start 130.659 65.7315) (end 130.683 65.7075) (width 0.5) (layer F.Cu) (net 3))
 (segment (start 130.659 68.751) (end 130.659 65.7315) (width 0.5) (layer F.Cu) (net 3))
 (via (at 133.35 59.689984) (size 0.8) (drill 0.4) (layers F.Cu B.Cu) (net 3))
 (segment (start 133.35 67.31) (end 133.35 59.689984) (width 0.5) (layer B.Cu) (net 3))
 (segment (start 130.27 58.42) (end 132.080016 58.42) (width 0.5) (layer F.Cu) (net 3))
 (segment (start 132.080016 58.42) (end 133.35 59.689984) (width 0.5) (layer F.Cu) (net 3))
 (segment (start 69.5454 60.1472) (end 69.5454 55.5754) (width 0.5) (layer F.Cu) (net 4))
 (segment (start 69.5454 55.5754) (end 67.31 53.34) (width 0.5) (layer F.Cu) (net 4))
 (segment (start 67.31 53.34) (end 65.42 53.34) (width 0.5) (layer F.Cu) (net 4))
 (via (at 63.5 69.85) (size 0.8) (drill 0.4) (layers F.Cu B.Cu) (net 4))
 (segment (start 61.7728 71.5772) (end 63.5 69.85) (width 0.5) (layer F.Cu) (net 4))
 (segment (start 60.0454 71.5772) (end 61.7728 71.5772) (width 0.5) (layer F.Cu) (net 4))
 (segment (start 64.77 68.58) (end 64.77 60.96) (width 0.5) (layer B.Cu) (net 4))
 (via (at 64.77 60.96) (size 0.8) (drill 0.4) (layers F.Cu B.Cu) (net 4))
 (segment (start 63.5 69.85) (end 64.77 68.58) (width 0.5) (layer B.Cu) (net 4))
 (segment (start 66.8528 60.1472) (end 69.5454 60.1472) (width 0.5) (layer F.Cu) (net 4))
 (segment (start 66.04 60.96) (end 66.8528 60.1472) (width 0.5) (layer F.Cu) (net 4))
 (segment (start 64.77 60.96) (end 66.04 60.96) (width 0.5) (layer F.Cu) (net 4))
 (via (at 78.74 55.88) (size 0.8) (drill 0.4) (layers F.Cu B.Cu) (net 4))
 (segment (start 76.2 53.34) (end 78.74 55.88) (width 0.5) (layer F.Cu) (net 4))
 (segment (start 67.31 53.34) (end 76.2 53.34) (width 0.5) (layer F.Cu) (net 4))
 (via (at 120.65 82.55) (size 0.8) (drill 0.4) (layers F.Cu B.Cu) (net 4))
 (segment (start 121.49 77.5) (end 123.19 77.5) (width 0.5) (layer F.Cu) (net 4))
 (segment (start 120.65 78.34) (end 121.49 77.5) (width 0.5) (layer F.Cu) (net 4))
 (segment (start 120.65 82.55) (end 120.65 78.34) (width 0.5) (layer F.Cu) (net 4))
 (segment (start 60.0454 74.0154) (end 60.0454 71.5772) (width 0.5) (layer F.Cu) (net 4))
 (segment (start 60.0454 74.0154) (end 60.96 74.93) (width 0.5) (layer F.Cu) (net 4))
 (segment (start 60.96 74.93) (end 64.12 74.93) (width 0.5) (layer F.Cu) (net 4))
 (segment (start 119.38 86.36) (end 120.65 85.09) (width 0.5) (layer B.Cu) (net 4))
 (segment (start 120.65 85.09) (end 120.65 82.55) (width 0.5) (layer B.Cu) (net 4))
 (segment (start 80.645 86.36) (end 119.38 86.36) (width 0.5) (layer B.Cu) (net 4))
 (segment (start 78.74 84.455) (end 80.645 86.36) (width 0.5) (layer B.Cu) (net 4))
 (segment (start 78.74 55.88) (end 78.74 84.455) (width 0.5) (layer B.Cu) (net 4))
 (segment (start 123.19 77.5) (end 123.19 62.23) (width 0.5) (layer F.Cu) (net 4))
 (segment (start 64.12 53.34) (end 62.23 53.34) (width 0.5) (layer F.Cu) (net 6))
 (segment (start 60.0454 55.5246) (end 62.23 53.34) (width 0.5) (layer F.Cu) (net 6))
 (segment (start 60.0454 60.1472) (end 60.0454 55.5246) (width 0.5) (layer F.Cu) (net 6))
 (segment (start 69.5454 73.9646) (end 69.5454 71.5772) (width 0.5) (layer F.Cu) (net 5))
 (segment (start 69.5454 73.9646) (end 68.58 74.93) (width 0.5) (layer F.Cu) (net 5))
 (segment (start 68.58 74.93) (end 65.42 74.93) (width 0.5) (layer F.Cu) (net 5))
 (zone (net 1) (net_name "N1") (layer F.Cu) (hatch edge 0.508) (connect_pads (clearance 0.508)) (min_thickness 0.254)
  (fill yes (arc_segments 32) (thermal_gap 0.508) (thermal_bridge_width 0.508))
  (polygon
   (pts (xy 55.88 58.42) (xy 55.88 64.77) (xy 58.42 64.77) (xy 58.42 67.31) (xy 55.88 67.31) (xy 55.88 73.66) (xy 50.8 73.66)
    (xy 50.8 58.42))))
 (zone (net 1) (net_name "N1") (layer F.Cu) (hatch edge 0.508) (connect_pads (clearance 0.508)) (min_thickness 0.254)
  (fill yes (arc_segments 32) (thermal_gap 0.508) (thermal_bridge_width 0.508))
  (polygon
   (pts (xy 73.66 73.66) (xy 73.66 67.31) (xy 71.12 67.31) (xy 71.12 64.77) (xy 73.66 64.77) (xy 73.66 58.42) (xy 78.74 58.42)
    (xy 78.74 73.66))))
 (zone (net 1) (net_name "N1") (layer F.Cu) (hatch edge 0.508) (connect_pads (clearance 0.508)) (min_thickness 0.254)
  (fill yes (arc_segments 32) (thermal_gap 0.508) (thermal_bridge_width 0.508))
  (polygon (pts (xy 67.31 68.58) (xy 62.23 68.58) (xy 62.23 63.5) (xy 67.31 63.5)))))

